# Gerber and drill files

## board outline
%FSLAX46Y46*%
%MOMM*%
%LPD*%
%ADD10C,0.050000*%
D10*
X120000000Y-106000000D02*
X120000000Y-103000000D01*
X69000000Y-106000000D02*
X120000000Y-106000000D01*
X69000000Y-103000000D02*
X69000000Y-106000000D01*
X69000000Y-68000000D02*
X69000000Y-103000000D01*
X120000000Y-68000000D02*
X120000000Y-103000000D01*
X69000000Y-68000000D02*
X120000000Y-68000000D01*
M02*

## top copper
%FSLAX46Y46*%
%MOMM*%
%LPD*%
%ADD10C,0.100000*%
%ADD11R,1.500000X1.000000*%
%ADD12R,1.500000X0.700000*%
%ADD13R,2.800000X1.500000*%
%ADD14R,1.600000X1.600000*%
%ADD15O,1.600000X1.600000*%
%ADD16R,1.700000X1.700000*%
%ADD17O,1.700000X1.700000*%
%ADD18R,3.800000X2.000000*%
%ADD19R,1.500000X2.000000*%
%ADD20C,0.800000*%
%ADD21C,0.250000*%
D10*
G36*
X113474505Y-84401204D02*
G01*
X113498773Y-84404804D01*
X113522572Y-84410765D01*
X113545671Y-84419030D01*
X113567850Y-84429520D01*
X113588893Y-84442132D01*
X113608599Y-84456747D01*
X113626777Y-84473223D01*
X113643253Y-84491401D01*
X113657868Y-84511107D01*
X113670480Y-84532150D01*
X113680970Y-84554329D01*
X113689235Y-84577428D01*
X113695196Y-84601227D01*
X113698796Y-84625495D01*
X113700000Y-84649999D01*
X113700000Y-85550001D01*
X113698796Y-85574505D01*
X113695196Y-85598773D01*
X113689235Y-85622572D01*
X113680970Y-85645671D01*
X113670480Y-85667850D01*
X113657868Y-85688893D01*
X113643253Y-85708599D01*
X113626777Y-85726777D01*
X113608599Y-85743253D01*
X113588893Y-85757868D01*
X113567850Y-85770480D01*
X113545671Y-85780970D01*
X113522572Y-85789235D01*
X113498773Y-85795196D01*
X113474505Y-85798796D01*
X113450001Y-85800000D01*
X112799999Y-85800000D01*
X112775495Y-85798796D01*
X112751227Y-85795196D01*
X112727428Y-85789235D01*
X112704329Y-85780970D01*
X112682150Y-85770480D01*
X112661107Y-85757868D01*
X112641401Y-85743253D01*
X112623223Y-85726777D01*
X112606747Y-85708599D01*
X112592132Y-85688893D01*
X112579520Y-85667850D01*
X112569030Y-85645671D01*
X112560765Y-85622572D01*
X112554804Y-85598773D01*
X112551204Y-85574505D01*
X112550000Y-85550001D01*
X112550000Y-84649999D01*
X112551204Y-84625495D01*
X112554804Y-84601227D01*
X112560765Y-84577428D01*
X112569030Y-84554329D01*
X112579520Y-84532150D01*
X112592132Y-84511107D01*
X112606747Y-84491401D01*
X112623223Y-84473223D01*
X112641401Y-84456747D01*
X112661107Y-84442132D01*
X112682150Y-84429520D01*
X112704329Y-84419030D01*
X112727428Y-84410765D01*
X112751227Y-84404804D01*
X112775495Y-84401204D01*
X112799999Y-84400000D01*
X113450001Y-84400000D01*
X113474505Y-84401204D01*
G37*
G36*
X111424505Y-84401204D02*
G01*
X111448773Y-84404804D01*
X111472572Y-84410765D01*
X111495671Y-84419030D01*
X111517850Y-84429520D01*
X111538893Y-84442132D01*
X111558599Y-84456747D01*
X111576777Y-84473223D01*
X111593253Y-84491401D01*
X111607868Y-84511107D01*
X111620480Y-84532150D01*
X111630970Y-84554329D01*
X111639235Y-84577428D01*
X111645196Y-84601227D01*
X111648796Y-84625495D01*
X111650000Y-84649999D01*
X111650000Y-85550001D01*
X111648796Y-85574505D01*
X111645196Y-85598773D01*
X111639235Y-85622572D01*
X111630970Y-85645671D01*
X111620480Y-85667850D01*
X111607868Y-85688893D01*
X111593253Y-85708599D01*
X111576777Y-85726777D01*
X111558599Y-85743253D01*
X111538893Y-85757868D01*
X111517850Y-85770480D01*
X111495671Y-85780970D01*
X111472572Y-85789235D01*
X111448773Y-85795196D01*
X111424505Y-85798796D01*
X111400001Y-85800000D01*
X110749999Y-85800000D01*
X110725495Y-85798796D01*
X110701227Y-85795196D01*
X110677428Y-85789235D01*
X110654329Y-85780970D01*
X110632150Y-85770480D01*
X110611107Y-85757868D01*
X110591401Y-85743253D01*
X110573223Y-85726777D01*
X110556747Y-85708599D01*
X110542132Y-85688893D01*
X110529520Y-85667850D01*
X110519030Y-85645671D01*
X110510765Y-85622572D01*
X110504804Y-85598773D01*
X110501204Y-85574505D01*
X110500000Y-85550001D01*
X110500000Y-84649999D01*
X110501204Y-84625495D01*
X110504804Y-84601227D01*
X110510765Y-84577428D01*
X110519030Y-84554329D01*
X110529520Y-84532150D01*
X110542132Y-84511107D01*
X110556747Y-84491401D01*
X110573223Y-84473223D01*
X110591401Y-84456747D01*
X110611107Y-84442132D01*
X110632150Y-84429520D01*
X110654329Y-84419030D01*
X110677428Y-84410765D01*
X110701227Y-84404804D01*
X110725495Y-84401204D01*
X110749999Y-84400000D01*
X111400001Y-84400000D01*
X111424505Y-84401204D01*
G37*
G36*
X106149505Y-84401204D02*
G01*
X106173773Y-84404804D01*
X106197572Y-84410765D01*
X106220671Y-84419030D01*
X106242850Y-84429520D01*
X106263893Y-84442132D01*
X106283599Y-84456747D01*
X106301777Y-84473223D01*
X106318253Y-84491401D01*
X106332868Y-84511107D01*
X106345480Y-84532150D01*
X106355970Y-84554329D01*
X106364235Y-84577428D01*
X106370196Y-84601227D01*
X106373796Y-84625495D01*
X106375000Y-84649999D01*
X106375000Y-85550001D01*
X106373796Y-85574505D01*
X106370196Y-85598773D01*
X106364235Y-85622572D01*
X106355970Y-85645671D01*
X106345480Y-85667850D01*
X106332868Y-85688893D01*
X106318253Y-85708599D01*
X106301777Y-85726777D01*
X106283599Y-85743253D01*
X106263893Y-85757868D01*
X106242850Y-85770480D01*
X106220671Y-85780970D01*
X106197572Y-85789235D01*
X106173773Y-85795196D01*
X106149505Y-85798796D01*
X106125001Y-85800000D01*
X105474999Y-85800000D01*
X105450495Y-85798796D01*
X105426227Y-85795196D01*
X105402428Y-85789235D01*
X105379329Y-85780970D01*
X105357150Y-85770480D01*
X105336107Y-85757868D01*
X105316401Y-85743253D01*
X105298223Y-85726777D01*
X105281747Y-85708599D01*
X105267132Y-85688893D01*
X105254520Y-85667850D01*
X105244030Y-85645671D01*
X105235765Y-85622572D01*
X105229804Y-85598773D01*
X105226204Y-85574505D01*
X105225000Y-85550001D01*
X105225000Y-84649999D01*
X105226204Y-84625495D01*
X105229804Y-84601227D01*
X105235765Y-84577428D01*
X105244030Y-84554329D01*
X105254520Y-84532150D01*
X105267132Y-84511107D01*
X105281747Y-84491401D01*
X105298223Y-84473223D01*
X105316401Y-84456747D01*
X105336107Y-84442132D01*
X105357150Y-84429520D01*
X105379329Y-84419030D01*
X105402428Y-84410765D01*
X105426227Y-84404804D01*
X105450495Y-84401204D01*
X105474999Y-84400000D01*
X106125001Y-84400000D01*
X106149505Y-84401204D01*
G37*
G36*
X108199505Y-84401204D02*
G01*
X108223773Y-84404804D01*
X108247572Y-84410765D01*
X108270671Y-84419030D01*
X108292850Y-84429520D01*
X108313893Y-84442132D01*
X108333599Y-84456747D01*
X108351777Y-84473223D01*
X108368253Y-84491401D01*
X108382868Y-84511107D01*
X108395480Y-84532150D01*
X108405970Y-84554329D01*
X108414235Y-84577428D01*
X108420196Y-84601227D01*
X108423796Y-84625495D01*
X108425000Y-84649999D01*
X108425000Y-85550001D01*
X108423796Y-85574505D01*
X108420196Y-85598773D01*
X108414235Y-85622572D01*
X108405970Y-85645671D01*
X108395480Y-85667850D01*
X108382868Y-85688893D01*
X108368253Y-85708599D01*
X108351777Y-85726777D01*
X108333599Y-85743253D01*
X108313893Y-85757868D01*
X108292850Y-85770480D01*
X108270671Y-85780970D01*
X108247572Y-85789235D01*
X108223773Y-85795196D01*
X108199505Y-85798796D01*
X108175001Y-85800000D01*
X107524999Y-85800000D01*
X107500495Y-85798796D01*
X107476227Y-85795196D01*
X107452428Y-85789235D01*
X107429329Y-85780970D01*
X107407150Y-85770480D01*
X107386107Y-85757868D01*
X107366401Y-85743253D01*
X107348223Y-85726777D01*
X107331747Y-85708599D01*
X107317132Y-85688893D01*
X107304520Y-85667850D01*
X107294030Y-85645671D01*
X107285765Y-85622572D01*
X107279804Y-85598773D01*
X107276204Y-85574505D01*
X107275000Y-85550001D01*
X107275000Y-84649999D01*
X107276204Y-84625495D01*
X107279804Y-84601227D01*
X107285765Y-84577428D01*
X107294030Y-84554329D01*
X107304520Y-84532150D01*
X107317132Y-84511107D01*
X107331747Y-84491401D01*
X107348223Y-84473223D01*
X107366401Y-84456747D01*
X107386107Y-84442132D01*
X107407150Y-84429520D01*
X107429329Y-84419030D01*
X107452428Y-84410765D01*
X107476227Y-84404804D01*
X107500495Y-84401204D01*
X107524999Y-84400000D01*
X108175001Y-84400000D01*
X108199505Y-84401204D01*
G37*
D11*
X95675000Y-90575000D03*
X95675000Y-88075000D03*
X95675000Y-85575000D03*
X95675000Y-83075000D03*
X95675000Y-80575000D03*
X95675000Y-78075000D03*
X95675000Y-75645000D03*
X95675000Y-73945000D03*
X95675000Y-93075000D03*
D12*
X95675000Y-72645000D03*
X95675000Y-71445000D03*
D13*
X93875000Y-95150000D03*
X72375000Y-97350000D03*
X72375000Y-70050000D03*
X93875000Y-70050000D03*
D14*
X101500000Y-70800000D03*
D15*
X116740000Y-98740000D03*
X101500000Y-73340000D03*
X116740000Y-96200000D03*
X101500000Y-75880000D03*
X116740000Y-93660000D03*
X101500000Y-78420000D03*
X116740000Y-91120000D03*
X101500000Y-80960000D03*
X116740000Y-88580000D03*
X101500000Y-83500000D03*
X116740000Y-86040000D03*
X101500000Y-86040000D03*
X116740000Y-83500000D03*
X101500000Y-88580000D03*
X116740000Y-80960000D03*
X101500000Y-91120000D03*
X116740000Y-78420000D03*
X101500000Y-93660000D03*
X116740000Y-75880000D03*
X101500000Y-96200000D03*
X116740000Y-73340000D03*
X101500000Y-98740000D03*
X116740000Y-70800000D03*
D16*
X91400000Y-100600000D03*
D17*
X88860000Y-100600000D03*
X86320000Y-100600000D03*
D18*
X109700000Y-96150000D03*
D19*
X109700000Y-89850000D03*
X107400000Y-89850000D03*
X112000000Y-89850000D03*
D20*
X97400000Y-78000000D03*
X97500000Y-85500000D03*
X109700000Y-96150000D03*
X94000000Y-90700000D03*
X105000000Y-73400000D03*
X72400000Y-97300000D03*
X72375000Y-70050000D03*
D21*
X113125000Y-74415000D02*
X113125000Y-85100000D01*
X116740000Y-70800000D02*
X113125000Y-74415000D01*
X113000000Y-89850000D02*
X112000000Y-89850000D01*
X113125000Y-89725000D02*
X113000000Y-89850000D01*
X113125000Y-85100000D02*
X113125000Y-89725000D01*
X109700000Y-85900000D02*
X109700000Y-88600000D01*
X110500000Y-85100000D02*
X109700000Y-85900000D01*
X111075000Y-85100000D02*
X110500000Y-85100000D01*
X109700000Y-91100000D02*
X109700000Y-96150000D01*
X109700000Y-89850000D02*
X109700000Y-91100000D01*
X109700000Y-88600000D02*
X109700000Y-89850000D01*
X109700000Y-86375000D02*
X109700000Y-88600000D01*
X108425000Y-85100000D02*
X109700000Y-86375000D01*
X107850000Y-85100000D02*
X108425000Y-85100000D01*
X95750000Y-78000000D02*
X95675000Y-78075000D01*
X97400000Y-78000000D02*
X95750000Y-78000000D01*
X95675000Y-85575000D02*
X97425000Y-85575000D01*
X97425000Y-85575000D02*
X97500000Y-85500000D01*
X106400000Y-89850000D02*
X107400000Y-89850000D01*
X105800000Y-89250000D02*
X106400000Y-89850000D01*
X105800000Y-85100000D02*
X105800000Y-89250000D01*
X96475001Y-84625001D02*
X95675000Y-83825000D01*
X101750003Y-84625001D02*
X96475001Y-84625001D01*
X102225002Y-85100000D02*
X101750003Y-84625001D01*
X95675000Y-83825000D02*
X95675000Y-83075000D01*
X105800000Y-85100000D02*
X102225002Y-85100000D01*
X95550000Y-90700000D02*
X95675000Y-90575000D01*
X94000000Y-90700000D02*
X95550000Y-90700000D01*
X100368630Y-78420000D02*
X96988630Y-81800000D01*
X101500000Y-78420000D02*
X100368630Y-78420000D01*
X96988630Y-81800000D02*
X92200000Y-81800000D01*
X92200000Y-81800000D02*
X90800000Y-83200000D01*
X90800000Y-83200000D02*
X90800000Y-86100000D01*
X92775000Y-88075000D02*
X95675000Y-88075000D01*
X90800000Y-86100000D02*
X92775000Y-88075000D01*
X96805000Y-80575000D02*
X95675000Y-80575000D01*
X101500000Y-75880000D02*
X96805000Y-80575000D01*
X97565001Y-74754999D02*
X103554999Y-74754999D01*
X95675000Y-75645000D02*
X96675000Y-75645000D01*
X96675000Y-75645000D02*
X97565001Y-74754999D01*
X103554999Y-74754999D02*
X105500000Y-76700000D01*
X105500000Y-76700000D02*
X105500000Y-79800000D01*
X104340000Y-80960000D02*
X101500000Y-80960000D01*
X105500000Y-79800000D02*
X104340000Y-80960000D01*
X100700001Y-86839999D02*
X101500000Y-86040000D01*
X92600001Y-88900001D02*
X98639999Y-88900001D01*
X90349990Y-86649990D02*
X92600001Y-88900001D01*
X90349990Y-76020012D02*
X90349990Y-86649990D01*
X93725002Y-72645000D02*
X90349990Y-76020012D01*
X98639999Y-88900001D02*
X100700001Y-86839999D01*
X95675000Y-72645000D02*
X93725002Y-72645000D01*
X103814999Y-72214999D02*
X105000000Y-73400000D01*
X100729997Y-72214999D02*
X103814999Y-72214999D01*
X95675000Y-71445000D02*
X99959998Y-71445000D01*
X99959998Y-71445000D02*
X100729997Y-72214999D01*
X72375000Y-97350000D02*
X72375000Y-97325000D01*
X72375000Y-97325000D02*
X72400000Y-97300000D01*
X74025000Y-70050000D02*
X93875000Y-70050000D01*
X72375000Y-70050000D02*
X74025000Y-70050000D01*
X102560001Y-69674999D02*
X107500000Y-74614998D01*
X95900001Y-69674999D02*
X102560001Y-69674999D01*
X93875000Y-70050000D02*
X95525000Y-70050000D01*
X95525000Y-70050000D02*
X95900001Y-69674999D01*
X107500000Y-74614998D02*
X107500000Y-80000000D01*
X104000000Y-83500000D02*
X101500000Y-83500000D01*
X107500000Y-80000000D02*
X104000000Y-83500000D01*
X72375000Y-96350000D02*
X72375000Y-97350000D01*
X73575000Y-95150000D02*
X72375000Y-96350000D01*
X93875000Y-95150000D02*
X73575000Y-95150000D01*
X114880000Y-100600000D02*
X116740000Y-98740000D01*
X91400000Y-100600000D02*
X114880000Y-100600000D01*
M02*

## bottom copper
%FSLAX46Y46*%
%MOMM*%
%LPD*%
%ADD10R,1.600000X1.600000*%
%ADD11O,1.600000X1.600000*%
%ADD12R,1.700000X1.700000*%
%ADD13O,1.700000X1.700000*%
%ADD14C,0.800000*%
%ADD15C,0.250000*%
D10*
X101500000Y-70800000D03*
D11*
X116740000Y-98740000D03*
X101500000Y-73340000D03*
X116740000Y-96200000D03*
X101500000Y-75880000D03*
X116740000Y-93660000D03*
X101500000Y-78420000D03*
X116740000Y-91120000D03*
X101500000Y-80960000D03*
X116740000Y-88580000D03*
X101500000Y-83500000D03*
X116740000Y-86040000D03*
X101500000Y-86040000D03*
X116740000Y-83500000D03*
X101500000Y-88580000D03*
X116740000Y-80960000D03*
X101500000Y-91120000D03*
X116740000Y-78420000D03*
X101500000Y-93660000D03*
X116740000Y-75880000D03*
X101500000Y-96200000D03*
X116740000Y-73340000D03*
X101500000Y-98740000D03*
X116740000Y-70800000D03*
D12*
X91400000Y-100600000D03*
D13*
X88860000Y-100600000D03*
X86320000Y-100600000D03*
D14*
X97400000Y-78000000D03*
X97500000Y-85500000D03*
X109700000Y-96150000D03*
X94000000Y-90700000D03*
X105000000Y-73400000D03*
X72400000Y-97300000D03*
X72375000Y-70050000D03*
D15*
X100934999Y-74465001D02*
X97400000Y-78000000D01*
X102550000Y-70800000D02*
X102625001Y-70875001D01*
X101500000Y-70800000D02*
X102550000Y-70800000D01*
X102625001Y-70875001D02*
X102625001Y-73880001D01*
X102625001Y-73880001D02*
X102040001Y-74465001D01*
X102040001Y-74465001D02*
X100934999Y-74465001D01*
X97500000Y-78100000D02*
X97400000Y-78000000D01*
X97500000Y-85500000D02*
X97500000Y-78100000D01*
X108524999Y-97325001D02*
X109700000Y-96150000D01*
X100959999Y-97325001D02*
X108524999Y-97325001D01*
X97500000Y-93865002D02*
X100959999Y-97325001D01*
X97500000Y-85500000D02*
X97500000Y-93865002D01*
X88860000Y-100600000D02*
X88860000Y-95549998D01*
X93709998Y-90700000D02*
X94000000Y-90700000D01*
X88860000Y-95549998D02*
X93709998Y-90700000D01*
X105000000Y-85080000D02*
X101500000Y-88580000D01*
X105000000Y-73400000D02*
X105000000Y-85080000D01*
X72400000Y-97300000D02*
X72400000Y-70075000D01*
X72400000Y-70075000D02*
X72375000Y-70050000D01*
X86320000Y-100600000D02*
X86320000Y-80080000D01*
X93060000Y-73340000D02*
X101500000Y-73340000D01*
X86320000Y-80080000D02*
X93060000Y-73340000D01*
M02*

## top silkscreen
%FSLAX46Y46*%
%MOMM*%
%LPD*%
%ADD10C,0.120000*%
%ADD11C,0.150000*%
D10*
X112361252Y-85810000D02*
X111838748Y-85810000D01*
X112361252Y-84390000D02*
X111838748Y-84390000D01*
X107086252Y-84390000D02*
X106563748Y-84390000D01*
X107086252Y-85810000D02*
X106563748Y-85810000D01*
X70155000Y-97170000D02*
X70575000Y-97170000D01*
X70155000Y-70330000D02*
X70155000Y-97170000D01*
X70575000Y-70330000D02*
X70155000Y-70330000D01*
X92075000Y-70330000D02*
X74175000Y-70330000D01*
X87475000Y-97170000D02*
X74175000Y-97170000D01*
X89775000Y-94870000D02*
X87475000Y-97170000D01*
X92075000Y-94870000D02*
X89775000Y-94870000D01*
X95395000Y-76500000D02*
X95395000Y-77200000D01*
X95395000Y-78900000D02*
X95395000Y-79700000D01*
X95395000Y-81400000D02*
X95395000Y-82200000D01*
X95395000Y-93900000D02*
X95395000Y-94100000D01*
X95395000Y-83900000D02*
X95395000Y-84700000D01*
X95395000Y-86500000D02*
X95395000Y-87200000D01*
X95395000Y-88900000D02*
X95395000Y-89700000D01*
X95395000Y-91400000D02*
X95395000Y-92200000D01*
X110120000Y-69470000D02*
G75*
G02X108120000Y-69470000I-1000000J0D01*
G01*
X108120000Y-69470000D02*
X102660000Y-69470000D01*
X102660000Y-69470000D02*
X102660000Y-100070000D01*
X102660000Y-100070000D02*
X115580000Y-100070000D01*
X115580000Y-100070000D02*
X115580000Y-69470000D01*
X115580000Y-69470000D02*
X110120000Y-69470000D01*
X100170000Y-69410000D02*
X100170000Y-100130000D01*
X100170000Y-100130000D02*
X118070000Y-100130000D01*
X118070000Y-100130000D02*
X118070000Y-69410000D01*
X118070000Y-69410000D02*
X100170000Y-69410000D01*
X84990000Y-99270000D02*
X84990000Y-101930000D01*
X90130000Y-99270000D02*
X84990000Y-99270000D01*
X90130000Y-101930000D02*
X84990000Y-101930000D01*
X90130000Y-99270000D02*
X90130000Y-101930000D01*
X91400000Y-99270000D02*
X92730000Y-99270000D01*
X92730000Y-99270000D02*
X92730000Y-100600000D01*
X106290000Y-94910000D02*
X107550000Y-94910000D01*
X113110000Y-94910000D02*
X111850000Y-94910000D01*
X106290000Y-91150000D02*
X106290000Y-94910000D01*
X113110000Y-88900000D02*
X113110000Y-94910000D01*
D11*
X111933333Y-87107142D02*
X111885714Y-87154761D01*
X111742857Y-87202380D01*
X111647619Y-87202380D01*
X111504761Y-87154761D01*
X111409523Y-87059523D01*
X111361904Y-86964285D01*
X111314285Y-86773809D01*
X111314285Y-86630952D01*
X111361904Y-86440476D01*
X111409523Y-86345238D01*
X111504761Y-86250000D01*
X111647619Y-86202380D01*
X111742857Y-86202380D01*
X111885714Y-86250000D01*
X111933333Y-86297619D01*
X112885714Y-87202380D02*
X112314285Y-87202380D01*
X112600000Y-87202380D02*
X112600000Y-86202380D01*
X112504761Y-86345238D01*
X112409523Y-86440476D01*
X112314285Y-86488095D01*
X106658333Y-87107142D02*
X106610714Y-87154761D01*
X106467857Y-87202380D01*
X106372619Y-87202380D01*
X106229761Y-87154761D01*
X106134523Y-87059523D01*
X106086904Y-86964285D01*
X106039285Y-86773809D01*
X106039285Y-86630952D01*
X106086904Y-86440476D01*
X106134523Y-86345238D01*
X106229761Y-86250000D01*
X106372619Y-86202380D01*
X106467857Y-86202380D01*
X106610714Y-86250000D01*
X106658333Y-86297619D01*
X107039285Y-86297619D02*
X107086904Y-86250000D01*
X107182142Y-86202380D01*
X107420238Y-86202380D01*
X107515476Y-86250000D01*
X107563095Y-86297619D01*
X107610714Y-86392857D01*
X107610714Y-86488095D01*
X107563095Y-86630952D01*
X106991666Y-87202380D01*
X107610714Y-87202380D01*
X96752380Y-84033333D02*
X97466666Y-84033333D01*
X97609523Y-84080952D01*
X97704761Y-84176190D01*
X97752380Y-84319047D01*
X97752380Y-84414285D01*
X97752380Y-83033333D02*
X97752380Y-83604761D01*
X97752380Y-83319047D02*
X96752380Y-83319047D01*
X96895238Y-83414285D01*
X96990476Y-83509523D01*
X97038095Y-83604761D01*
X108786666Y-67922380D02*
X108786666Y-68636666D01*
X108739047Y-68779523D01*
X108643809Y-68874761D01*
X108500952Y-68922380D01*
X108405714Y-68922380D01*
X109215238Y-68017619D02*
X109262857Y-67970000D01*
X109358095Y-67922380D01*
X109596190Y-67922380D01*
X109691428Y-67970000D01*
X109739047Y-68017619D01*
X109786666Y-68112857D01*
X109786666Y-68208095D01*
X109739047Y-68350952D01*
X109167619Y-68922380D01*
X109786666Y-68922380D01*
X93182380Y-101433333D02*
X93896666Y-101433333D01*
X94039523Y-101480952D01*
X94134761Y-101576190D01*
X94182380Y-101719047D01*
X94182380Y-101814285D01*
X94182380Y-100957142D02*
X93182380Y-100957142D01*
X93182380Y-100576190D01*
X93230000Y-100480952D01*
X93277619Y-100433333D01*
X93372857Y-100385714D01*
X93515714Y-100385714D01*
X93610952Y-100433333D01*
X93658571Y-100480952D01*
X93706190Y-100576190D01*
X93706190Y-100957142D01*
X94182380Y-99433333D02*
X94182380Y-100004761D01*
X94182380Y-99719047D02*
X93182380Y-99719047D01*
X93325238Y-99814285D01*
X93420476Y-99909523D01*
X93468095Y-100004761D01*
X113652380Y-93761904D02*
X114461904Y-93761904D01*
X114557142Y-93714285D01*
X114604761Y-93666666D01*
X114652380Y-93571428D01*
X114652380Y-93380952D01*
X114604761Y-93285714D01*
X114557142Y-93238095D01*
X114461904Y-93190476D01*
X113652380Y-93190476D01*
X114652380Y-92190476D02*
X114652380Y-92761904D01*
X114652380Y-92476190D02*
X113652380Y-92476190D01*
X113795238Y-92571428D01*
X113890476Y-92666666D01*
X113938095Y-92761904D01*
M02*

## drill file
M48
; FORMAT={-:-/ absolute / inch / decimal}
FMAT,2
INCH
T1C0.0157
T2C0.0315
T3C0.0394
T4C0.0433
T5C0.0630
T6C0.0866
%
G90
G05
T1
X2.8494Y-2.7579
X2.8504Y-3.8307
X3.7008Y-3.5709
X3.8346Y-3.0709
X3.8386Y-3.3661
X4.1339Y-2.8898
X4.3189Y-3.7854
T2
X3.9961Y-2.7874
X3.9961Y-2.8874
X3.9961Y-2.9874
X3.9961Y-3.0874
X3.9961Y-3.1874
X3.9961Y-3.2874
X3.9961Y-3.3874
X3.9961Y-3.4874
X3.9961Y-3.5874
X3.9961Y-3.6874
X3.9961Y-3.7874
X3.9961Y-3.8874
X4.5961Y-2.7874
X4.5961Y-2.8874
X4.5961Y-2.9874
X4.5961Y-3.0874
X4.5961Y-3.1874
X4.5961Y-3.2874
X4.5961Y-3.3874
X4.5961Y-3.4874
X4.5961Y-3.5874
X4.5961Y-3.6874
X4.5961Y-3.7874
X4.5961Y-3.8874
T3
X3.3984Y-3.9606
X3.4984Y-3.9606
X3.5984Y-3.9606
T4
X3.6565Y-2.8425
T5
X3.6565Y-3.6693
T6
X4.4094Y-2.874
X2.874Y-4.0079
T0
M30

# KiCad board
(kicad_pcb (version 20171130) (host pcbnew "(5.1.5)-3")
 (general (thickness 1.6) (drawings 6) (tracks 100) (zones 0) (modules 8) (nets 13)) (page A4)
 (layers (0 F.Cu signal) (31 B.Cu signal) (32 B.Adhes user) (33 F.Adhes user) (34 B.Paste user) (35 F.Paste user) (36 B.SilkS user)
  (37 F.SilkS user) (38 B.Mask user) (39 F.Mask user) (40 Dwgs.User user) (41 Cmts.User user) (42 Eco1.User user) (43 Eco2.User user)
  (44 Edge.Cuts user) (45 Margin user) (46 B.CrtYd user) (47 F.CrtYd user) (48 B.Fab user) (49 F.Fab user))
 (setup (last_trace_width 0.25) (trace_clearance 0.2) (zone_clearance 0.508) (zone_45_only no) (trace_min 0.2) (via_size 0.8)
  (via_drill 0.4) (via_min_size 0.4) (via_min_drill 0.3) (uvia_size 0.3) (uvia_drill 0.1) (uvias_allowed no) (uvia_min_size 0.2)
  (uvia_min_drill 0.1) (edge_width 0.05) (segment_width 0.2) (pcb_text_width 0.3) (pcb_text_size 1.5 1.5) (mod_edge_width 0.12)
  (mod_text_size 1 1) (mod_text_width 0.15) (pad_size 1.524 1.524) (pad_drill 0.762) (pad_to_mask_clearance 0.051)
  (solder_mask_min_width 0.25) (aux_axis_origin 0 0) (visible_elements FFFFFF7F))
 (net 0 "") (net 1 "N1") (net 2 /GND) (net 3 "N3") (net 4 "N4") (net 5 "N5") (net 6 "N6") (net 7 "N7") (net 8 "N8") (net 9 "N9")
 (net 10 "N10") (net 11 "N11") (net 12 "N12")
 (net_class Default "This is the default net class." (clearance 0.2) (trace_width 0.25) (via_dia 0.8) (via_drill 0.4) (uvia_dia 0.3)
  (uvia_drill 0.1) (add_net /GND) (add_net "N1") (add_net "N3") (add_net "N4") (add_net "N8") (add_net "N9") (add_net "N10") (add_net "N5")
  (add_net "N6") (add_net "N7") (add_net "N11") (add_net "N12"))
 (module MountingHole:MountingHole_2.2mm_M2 (layer F.Cu) (at 73 101.8)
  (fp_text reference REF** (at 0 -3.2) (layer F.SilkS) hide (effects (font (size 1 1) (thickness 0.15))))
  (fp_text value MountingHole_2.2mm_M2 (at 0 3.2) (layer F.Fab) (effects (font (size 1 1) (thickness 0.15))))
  (pad 1 np_thru_hole circle (at 0 0) (size 2.2 2.2) (drill 2.2) (layers *.Cu *.Mask)))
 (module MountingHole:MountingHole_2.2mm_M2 (layer F.Cu) (at 112 73)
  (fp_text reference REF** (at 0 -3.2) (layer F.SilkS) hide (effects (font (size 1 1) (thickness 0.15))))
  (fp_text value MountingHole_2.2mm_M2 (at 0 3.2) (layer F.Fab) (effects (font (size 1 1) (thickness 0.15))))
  (pad 1 np_thru_hole circle (at 0 0) (size 2.2 2.2) (drill 2.2) (layers *.Cu *.Mask)))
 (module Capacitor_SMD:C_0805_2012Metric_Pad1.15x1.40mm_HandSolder (layer F.Cu) (at 112.1 85.1 180)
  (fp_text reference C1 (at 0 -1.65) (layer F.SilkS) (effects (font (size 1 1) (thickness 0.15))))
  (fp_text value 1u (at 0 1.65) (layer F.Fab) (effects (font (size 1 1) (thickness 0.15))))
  (fp_line (start -0.261252 -0.71) (end 0.261252 -0.71) (layer F.SilkS) (width 0.12))
  (fp_line (start -0.261252 0.71) (end 0.261252 0.71) (layer F.SilkS) (width 0.12))
  (pad 1 smd roundrect (at -1.025 0 180) (size 1.15 1.4) (layers F.Cu F.Paste F.Mask) (roundrect_rratio 0.217391) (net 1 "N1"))
  (pad 2 smd roundrect (at 1.025 0 180) (size 1.15 1.4) (layers F.Cu F.Paste F.Mask) (roundrect_rratio 0.217391) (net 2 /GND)))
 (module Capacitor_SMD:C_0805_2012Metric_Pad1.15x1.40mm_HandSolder (layer F.Cu) (at 106.825 85.1 180)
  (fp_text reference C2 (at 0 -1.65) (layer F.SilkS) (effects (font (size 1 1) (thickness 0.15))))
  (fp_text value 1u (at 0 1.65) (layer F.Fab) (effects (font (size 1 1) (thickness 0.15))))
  (fp_line (start -0.261252 0.71) (end 0.261252 0.71) (layer F.SilkS) (width 0.12))
  (fp_line (start -0.261252 -0.71) (end 0.261252 -0.71) (layer F.SilkS) (width 0.12))
  (pad 2 smd roundrect (at 1.025 0 180) (size 1.15 1.4) (layers F.Cu F.Paste F.Mask) (roundrect_rratio 0.217391) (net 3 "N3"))
  (pad 1 smd roundrect (at -1.025 0 180) (size 1.15 1.4) (layers F.Cu F.Paste F.Mask) (roundrect_rratio 0.217391) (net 2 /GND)))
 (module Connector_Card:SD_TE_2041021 (layer F.Cu) (at 83.7 83.7 270)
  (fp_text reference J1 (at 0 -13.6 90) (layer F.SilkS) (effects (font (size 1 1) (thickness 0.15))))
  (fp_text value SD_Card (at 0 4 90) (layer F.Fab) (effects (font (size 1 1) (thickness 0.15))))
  (fp_line (start 13.47 13.545) (end 13.47 13.125) (layer F.SilkS) (width 0.12))
  (fp_line (start -13.37 13.545) (end 13.47 13.545) (layer F.SilkS) (width 0.12))
  (fp_line (start -13.37 13.125) (end -13.37 13.545) (layer F.SilkS) (width 0.12))
  (fp_line (start -13.37 -8.375) (end -13.37 9.525) (layer F.SilkS) (width 0.12))
  (fp_line (start 13.47 -3.775) (end 13.47 9.525) (layer F.SilkS) (width 0.12))
  (fp_line (start 11.17 -6.075) (end 13.47 -3.775) (layer F.SilkS) (width 0.12))
  (fp_line (start 11.17 -8.375) (end 11.17 -6.075) (layer F.SilkS) (width 0.12))
  (fp_line (start -7.2 -11.695) (end -6.5 -11.695) (layer F.SilkS) (width 0.12))
  (fp_line (start -4.8 -11.695) (end -4 -11.695) (layer F.SilkS) (width 0.12))
  (fp_line (start -2.3 -11.695) (end -1.5 -11.695) (layer F.SilkS) (width 0.12))
  (fp_line (start 10.2 -11.695) (end 10.4 -11.695) (layer F.SilkS) (width 0.12))
  (fp_line (start 0.2 -11.695) (end 1 -11.695) (layer F.SilkS) (width 0.12))
  (fp_line (start 2.8 -11.695) (end 3.5 -11.695) (layer F.SilkS) (width 0.12))
  (fp_line (start 5.2 -11.695) (end 6 -11.695) (layer F.SilkS) (width 0.12))
  (fp_line (start 7.7 -11.695) (end 8.5 -11.695) (layer F.SilkS) (width 0.12))
  (pad 1 smd rect (at 6.875 -11.975 270) (size 1 1.5) (layers F.Cu F.Paste F.Mask) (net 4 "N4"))
  (pad 2 smd rect (at 4.375 -11.975 270) (size 1 1.5) (layers F.Cu F.Paste F.Mask) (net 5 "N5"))
  (pad 3 smd rect (at 1.875 -11.975 270) (size 1 1.5) (layers F.Cu F.Paste F.Mask) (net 2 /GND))
  (pad 4 smd rect (at -0.625 -11.975 270) (size 1 1.5) (layers F.Cu F.Paste F.Mask) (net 3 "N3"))
  (pad 5 smd rect (at -3.125 -11.975 270) (size 1 1.5) (layers F.Cu F.Paste F.Mask) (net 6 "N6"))
  (pad 6 smd rect (at -5.625 -11.975 270) (size 1 1.5) (layers F.Cu F.Paste F.Mask) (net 2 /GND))
  (pad 7 smd rect (at -8.055 -11.975 270) (size 1 1.5) (layers F.Cu F.Paste F.Mask) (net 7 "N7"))
  (pad 8 smd rect (at -9.755 -11.975 270) (size 1 1.5) (layers F.Cu F.Paste F.Mask))
  (pad 9 smd rect (at 9.375 -11.975 270) (size 1 1.5) (layers F.Cu F.Paste F.Mask))
  (pad 10 smd rect (at -11.055 -11.975 270) (size 0.7 1.5) (layers F.Cu F.Paste F.Mask) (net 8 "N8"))
  (pad 11 smd rect (at -12.255 -11.975 270) (size 0.7 1.5) (layers F.Cu F.Paste F.Mask) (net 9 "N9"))
  (pad "" np_thru_hole circle (at 9.5 -9.175 270) (size 1.6 1.6) (drill 1.6) (layers *.Cu *.Mask))
  (pad "" np_thru_hole circle (at -11.5 -9.175 270) (size 1.1 1.1) (drill 1.1) (layers *.Cu *.Mask))
  (pad 12 smd rect (at 11.45 -10.175 270) (size 1.5 2.8) (layers F.Cu F.Paste F.Mask) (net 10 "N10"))
  (pad 12 smd rect (at 13.65 11.325 270) (size 1.5 2.8) (layers F.Cu F.Paste F.Mask) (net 10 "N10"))
  (pad 12 smd rect (at -13.65 11.325 270) (size 1.5 2.8) (layers F.Cu F.Paste F.Mask) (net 10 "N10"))
  (pad 12 smd rect (at -13.65 -10.175 270) (size 1.5 2.8) (layers F.Cu F.Paste F.Mask) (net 10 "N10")))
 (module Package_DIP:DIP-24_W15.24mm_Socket (layer F.Cu) (at 101.5 70.8)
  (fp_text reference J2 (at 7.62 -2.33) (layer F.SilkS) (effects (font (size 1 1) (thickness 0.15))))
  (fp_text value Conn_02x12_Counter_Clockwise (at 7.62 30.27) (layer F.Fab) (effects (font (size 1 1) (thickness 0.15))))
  (fp_arc (start 7.62 -1.33) (end 6.62 -1.33) (angle -180) (layer F.SilkS) (width 0.12))
  (fp_line (start 6.62 -1.33) (end 1.16 -1.33) (layer F.SilkS) (width 0.12))
  (fp_line (start 1.16 -1.33) (end 1.16 29.27) (layer F.SilkS) (width 0.12))
  (fp_line (start 1.16 29.27) (end 14.08 29.27) (layer F.SilkS) (width 0.12))
  (fp_line (start 14.08 29.27) (end 14.08 -1.33) (layer F.SilkS) (width 0.12))
  (fp_line (start 14.08 -1.33) (end 8.62 -1.33) (layer F.SilkS) (width 0.12))
  (fp_line (start -1.33 -1.39) (end -1.33 29.33) (layer F.SilkS) (width 0.12))
  (fp_line (start -1.33 29.33) (end 16.57 29.33) (layer F.SilkS) (width 0.12))
  (fp_line (start 16.57 29.33) (end 16.57 -1.39) (layer F.SilkS) (width 0.12))
  (fp_line (start 16.57 -1.39) (end -1.33 -1.39) (layer F.SilkS) (width 0.12))
  (pad 1 thru_hole rect (at 0 0) (size 1.6 1.6) (drill 0.8) (layers *.Cu *.Mask) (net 2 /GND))
  (pad 13 thru_hole oval (at 15.24 27.94) (size 1.6 1.6) (drill 0.8) (layers *.Cu *.Mask) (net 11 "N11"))
  (pad 2 thru_hole oval (at 0 2.54) (size 1.6 1.6) (drill 0.8) (layers *.Cu *.Mask) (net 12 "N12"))
  (pad 14 thru_hole oval (at 15.24 25.4) (size 1.6 1.6) (drill 0.8) (layers *.Cu *.Mask))
  (pad 3 thru_hole oval (at 0 5.08) (size 1.6 1.6) (drill 0.8) (layers *.Cu *.Mask) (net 6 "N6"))
  (pad 15 thru_hole oval (at 15.24 22.86) (size 1.6 1.6) (drill 0.8) (layers *.Cu *.Mask))
  (pad 4 thru_hole oval (at 0 7.62) (size 1.6 1.6) (drill 0.8) (layers *.Cu *.Mask) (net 5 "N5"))
  (pad 16 thru_hole oval (at 15.24 20.32) (size 1.6 1.6) (drill 0.8) (layers *.Cu *.Mask))
  (pad 5 thru_hole oval (at 0 10.16) (size 1.6 1.6) (drill 0.8) (layers *.Cu *.Mask) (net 7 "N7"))
  (pad 17 thru_hole oval (at 15.24 17.78) (size 1.6 1.6) (drill 0.8) (layers *.Cu *.Mask))
  (pad 6 thru_hole oval (at 0 12.7) (size 1.6 1.6) (drill 0.8) (layers *.Cu *.Mask) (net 10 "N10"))
  (pad 18 thru_hole oval (at 15.24 15.24) (size 1.6 1.6) (drill 0.8) (layers *.Cu *.Mask))
  (pad 7 thru_hole oval (at 0 15.24) (size 1.6 1.6) (drill 0.8) (layers *.Cu *.Mask) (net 8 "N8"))
  (pad 19 thru_hole oval (at 15.24 12.7) (size 1.6 1.6) (drill 0.8) (layers *.Cu *.Mask))
  (pad 8 thru_hole oval (at 0 17.78) (size 1.6 1.6) (drill 0.8) (layers *.Cu *.Mask) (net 9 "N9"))
  (pad 20 thru_hole oval (at 15.24 10.16) (size 1.6 1.6) (drill 0.8) (layers *.Cu *.Mask))
  (pad 9 thru_hole oval (at 0 20.32) (size 1.6 1.6) (drill 0.8) (layers *.Cu *.Mask))
  (pad 21 thru_hole oval (at 15.24 7.62) (size 1.6 1.6) (drill 0.8) (layers *.Cu *.Mask))
  (pad 10 thru_hole oval (at 0 22.86) (size 1.6 1.6) (drill 0.8) (layers *.Cu *.Mask))
  (pad 22 thru_hole oval (at 15.24 5.08) (size 1.6 1.6) (drill 0.8) (layers *.Cu *.Mask))
  (pad 11 thru_hole oval (at 0 25.4) (size 1.6 1.6) (drill 0.8) (layers *.Cu *.Mask))
  (pad 23 thru_hole oval (at 15.24 2.54) (size 1.6 1.6) (drill 0.8) (layers *.Cu *.Mask))
  (pad 12 thru_hole oval (at 0 27.94) (size 1.6 1.6) (drill 0.8) (layers *.Cu *.Mask))
  (pad 24 thru_hole oval (at 15.24 0) (size 1.6 1.6) (drill 0.8) (layers *.Cu *.Mask) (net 1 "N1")))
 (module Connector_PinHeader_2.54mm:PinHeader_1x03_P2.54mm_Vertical (layer F.Cu) (at 91.4 100.6 270)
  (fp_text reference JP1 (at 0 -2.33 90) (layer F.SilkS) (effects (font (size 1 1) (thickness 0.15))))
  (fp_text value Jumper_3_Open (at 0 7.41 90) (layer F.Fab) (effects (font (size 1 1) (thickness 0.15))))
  (fp_line (start -1.33 6.41) (end 1.33 6.41) (layer F.SilkS) (width 0.12))
  (fp_line (start -1.33 1.27) (end -1.33 6.41) (layer F.SilkS) (width 0.12))
  (fp_line (start 1.33 1.27) (end 1.33 6.41) (layer F.SilkS) (width 0.12))
  (fp_line (start -1.33 1.27) (end 1.33 1.27) (layer F.SilkS) (width 0.12))
  (fp_line (start -1.33 0) (end -1.33 -1.33) (layer F.SilkS) (width 0.12))
  (fp_line (start -1.33 -1.33) (end 0 -1.33) (layer F.SilkS) (width 0.12))
  (pad 1 thru_hole rect (at 0 0 270) (size 1.7 1.7) (drill 1) (layers *.Cu *.Mask) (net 11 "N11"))
  (pad 2 thru_hole oval (at 0 2.54 270) (size 1.7 1.7) (drill 1) (layers *.Cu *.Mask) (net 4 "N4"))
  (pad 3 thru_hole oval (at 0 5.08 270) (size 1.7 1.7) (drill 1) (layers *.Cu *.Mask) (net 12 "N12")))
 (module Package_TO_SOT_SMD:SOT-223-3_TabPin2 (layer F.Cu) (at 109.7 93 270)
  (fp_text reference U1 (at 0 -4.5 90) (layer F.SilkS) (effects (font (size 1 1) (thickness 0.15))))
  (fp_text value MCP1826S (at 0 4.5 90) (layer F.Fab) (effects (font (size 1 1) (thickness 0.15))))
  (fp_line (start 1.91 3.41) (end 1.91 2.15) (layer F.SilkS) (width 0.12))
  (fp_line (start 1.91 -3.41) (end 1.91 -2.15) (layer F.SilkS) (width 0.12))
  (fp_line (start -1.85 3.41) (end 1.91 3.41) (layer F.SilkS) (width 0.12))
  (fp_line (start -4.1 -3.41) (end 1.91 -3.41) (layer F.SilkS) (width 0.12))
  (pad 2 smd rect (at 3.15 0 270) (size 2 3.8) (layers F.Cu F.Paste F.Mask) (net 2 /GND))
  (pad 2 smd rect (at -3.15 0 270) (size 2 1.5) (layers F.Cu F.Paste F.Mask) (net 2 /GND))
  (pad 3 smd rect (at -3.15 2.3 270) (size 2 1.5) (layers F.Cu F.Paste F.Mask) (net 3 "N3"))
  (pad 1 smd rect (at -3.15 -2.3 270) (size 2 1.5) (layers F.Cu F.Paste F.Mask) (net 1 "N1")))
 (gr_line (start 120 106) (end 120 103) (layer Edge.Cuts) (width 0.05))
 (gr_line (start 69 106) (end 120 106) (layer Edge.Cuts) (width 0.05))
 (gr_line (start 69 103) (end 69 106) (layer Edge.Cuts) (width 0.05))
 (gr_line (start 69 68) (end 69 103) (layer Edge.Cuts) (width 0.05))
 (gr_line (start 120 68) (end 120 103) (layer Edge.Cuts) (width 0.05))
 (gr_line (start 69 68) (end 120 68) (layer Edge.Cuts) (width 0.05))
 (segment (start 113.125 74.415) (end 113.125 85.1) (width 0.25) (layer F.Cu) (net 1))
 (segment (start 116.74 70.8) (end 113.125 74.415) (width 0.25) (layer F.Cu) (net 1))
 (segment (start 113 89.85) (end 112 89.85) (width 0.25) (layer F.Cu) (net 1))
 (segment (start 113.125 89.725) (end 113 89.85) (width 0.25) (layer F.Cu) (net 1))
 (segment (start 113.125 85.1) (end 113.125 89.725) (width 0.25) (layer F.Cu) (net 1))
 (segment (start 109.7 85.9) (end 109.7 88.6) (width 0.25) (layer F.Cu) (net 2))
 (segment (start 110.5 85.1) (end 109.7 85.9) (width 0.25) (layer F.Cu) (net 2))
 (segment (start 111.075 85.1) (end 110.5 85.1) (width 0.25) (layer F.Cu) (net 2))
 (segment (start 109.7 91.1) (end 109.7 96.15) (width 0.25) (layer F.Cu) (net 2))
 (segment (start 109.7 89.85) (end 109.7 91.1) (width 0.25) (layer F.Cu) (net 2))
 (segment (start 109.7 88.6) (end 109.7 89.85) (width 0.25) (layer F.Cu) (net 2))
 (segment (start 109.7 86.375) (end 109.7 88.6) (width 0.25) (layer F.Cu) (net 2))
 (segment (start 108.425 85.1) (end 109.7 86.375) (width 0.25) (layer F.Cu) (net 2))
 (segment (start 107.85 85.1) (end 108.425 85.1) (width 0.25) (layer F.Cu) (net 2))
 (via (at 97.4 78) (size 0.8) (drill 0.4) (layers F.Cu B.Cu) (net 2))
 (segment (start 100.934999 74.465001) (end 97.4 78) (width 0.25) (layer B.Cu) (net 2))
 (segment (start 102.55 70.8) (end 102.625001 70.875001) (width 0.25) (layer B.Cu) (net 2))
 (segment (start 101.5 70.8) (end 102.55 70.8) (width 0.25) (layer B.Cu) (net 2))
 (segment (start 102.625001 70.875001) (end 102.625001 73.880001) (width 0.25) (layer B.Cu) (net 2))
 (segment (start 102.625001 73.880001) (end 102.040001 74.465001) (width 0.25) (layer B.Cu) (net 2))
 (segment (start 102.040001 74.465001) (end 100.934999 74.465001) (width 0.25) (layer B.Cu) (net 2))
 (segment (start 95.75 78) (end 95.675 78.075) (width 0.25) (layer F.Cu) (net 2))
 (segment (start 97.4 78) (end 95.75 78) (width 0.25) (layer F.Cu) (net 2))
 (segment (start 95.675 85.575) (end 97.425 85.575) (width 0.25) (layer F.Cu) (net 2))
 (via (at 97.5 85.5) (size 0.8) (drill 0.4) (layers F.Cu B.Cu) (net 2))
 (segment (start 97.425 85.575) (end 97.5 85.5) (width 0.25) (layer F.Cu) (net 2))
 (segment (start 97.5 78.1) (end 97.4 78) (width 0.25) (layer B.Cu) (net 2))
 (segment (start 97.5 85.5) (end 97.5 78.1) (width 0.25) (layer B.Cu) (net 2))
 (via (at 109.7 96.15) (size 0.8) (drill 0.4) (layers F.Cu B.Cu) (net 2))
 (segment (start 108.524999 97.325001) (end 109.7 96.15) (width 0.25) (layer B.Cu) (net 2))
 (segment (start 100.959999 97.325001) (end 108.524999 97.325001) (width 0.25) (layer B.Cu) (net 2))
 (segment (start 97.5 93.865002) (end 100.959999 97.325001) (width 0.25) (layer B.Cu) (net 2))
 (segment (start 97.5 85.5) (end 97.5 93.865002) (width 0.25) (layer B.Cu) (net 2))
 (segment (start 106.4 89.85) (end 107.4 89.85) (width 0.25) (layer F.Cu) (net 3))
 (segment (start 105.8 89.25) (end 106.4 89.85) (width 0.25) (layer F.Cu) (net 3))
 (segment (start 105.8 85.1) (end 105.8 89.25) (width 0.25) (layer F.Cu) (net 3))
 (segment (start 96.475001 84.625001) (end 95.675 83.825) (width 0.25) (layer F.Cu) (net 3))
 (segment (start 101.750003 84.625001) (end 96.475001 84.625001) (width 0.25) (layer F.Cu) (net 3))
 (segment (start 102.225002 85.1) (end 101.750003 84.625001) (width 0.25) (layer F.Cu) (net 3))
 (segment (start 95.675 83.825) (end 95.675 83.075) (width 0.25) (layer F.Cu) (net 3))
 (segment (start 105.8 85.1) (end 102.225002 85.1) (width 0.25) (layer F.Cu) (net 3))
 (via (at 94 90.7) (size 0.8) (drill 0.4) (layers F.Cu B.Cu) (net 4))
 (segment (start 88.86 100.6) (end 88.86 95.549998) (width 0.25) (layer B.Cu) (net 4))
 (segment (start 93.709998 90.7) (end 94 90.7) (width 0.25) (layer B.Cu) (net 4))
 (segment (start 88.86 95.549998) (end 93.709998 90.7) (width 0.25) (layer B.Cu) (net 4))
 (segment (start 95.55 90.7) (end 95.675 90.575) (width 0.25) (layer F.Cu) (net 4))
 (segment (start 94 90.7) (end 95.55 90.7) (width 0.25) (layer F.Cu) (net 4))
 (segment (start 100.36863 78.42) (end 96.98863 81.8) (width 0.25) (layer F.Cu) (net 5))
 (segment (start 101.5 78.42) (end 100.36863 78.42) (width 0.25) (layer F.Cu) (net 5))
 (segment (start 96.98863 81.8) (end 92.2 81.8) (width 0.25) (layer F.Cu) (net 5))
 (segment (start 92.2 81.8) (end 90.8 83.2) (width 0.25) (layer F.Cu) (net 5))
 (segment (start 90.8 83.2) (end 90.8 86.1) (width 0.25) (layer F.Cu) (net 5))
 (segment (start 92.775 88.075) (end 95.675 88.075) (width 0.25) (layer F.Cu) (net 5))
 (segment (start 90.8 86.1) (end 92.775 88.075) (width 0.25) (layer F.Cu) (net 5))
 (segment (start 96.805 80.575) (end 95.675 80.575) (width 0.25) (layer F.Cu) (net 6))
 (segment (start 101.5 75.88) (end 96.805 80.575) (width 0.25) (layer F.Cu) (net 6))
 (segment (start 97.565001 74.754999) (end 103.554999 74.754999) (width 0.25) (layer F.Cu) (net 7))
 (segment (start 95.675 75.645) (end 96.675 75.645) (width 0.25) (layer F.Cu) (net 7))
 (segment (start 96.675 75.645) (end 97.565001 74.754999) (width 0.25) (layer F.Cu) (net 7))
 (segment (start 103.554999 74.754999) (end 105.5 76.7) (width 0.25) (layer F.Cu) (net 7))
 (segment (start 105.5 76.7) (end 105.5 79.8) (width 0.25) (layer F.Cu) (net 7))
 (segment (start 104.34 80.96) (end 101.5 80.96) (width 0.25) (layer F.Cu) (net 7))
 (segment (start 105.5 79.8) (end 104.34 80.96) (width 0.25) (layer F.Cu) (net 7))
 (segment (start 100.700001 86.839999) (end 101.5 86.04) (width 0.25) (layer F.Cu) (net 8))
 (segment (start 92.600001 88.900001) (end 98.639999 88.900001) (width 0.25) (layer F.Cu) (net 8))
 (segment (start 90.34999 86.64999) (end 92.600001 88.900001) (width 0.25) (layer F.Cu) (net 8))
 (segment (start 90.34999 76.020012) (end 90.34999 86.64999) (width 0.25) (layer F.Cu) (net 8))
 (segment (start 93.725002 72.645) (end 90.34999 76.020012) (width 0.25) (layer F.Cu) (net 8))
 (segment (start 98.639999 88.900001) (end 100.700001 86.839999) (width 0.25) (layer F.Cu) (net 8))
 (segment (start 95.675 72.645) (end 93.725002 72.645) (width 0.25) (layer F.Cu) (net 8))
 (segment (start 103.814999 72.214999) (end 105 73.4) (width 0.25) (layer F.Cu) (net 9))
 (via (at 105 73.4) (size 0.8) (drill 0.4) (layers F.Cu B.Cu) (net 9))
 (segment (start 100.729997 72.214999) (end 103.814999 72.214999) (width 0.25) (layer F.Cu) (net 9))
 (segment (start 95.675 71.445) (end 99.959998 71.445) (width 0.25) (layer F.Cu) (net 9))
 (segment (start 99.959998 71.445) (end 100.729997 72.214999) (width 0.25) (layer F.Cu) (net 9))
 (segment (start 105 85.08) (end 101.5 88.58) (width 0.25) (layer B.Cu) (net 9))
 (segment (start 105 73.4) (end 105 85.08) (width 0.25) (layer B.Cu) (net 9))
 (via (at 72.4 97.3) (size 0.8) (drill 0.4) (layers F.Cu B.Cu) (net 10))
 (segment (start 72.375 97.35) (end 72.375 97.325) (width 0.25) (layer F.Cu) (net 10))
 (segment (start 72.375 97.325) (end 72.4 97.3) (width 0.25) (layer F.Cu) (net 10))
 (via (at 72.375 70.05) (size 0.8) (drill 0.4) (layers F.Cu B.Cu) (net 10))
 (segment (start 72.4 97.3) (end 72.4 70.075) (width 0.25) (layer B.Cu) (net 10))
 (segment (start 72.4 70.075) (end 72.375 70.05) (width 0.25) (layer B.Cu) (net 10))
 (segment (start 74.025 70.05) (end 93.875 70.05) (width 0.25) (layer F.Cu) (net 10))
 (segment (start 72.375 70.05) (end 74.025 70.05) (width 0.25) (layer F.Cu) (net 10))
 (segment (start 102.560001 69.674999) (end 107.5 74.614998) (width 0.25) (layer F.Cu) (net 10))
 (segment (start 95.900001 69.674999) (end 102.560001 69.674999) (width 0.25) (layer F.Cu) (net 10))
 (segment (start 93.875 70.05) (end 95.525 70.05) (width 0.25) (layer F.Cu) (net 10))
 (segment (start 95.525 70.05) (end 95.900001 69.674999) (width 0.25) (layer F.Cu) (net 10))
 (segment (start 107.5 74.614998) (end 107.5 80) (width 0.25) (layer F.Cu) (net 10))
 (segment (start 104 83.5) (end 101.5 83.5) (width 0.25) (layer F.Cu) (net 10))
 (segment (start 107.5 80) (end 104 83.5) (width 0.25) (layer F.Cu) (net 10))
 (segment (start 72.375 96.35) (end 72.375 97.35) (width 0.25) (layer F.Cu) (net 10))
 (segment (start 73.575 95.15) (end 72.375 96.35) (width 0.25) (layer F.Cu) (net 10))
 (segment (start 93.875 95.15) (end 73.575 95.15) (width 0.25) (layer F.Cu) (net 10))
 (segment (start 114.88 100.6) (end 116.74 98.74) (width 0.25) (layer F.Cu) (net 11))
 (segment (start 91.4 100.6) (end 114.88 100.6) (width 0.25) (layer F.Cu) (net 11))
 (segment (start 86.32 100.6) (end 86.32 80.08) (width 0.25) (layer B.Cu) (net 12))
 (segment (start 93.06 73.34) (end 101.5 73.34) (width 0.25) (layer B.Cu) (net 12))
 (segment (start 86.32 80.08) (end 93.06 73.34) (width 0.25) (layer B.Cu) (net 12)))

